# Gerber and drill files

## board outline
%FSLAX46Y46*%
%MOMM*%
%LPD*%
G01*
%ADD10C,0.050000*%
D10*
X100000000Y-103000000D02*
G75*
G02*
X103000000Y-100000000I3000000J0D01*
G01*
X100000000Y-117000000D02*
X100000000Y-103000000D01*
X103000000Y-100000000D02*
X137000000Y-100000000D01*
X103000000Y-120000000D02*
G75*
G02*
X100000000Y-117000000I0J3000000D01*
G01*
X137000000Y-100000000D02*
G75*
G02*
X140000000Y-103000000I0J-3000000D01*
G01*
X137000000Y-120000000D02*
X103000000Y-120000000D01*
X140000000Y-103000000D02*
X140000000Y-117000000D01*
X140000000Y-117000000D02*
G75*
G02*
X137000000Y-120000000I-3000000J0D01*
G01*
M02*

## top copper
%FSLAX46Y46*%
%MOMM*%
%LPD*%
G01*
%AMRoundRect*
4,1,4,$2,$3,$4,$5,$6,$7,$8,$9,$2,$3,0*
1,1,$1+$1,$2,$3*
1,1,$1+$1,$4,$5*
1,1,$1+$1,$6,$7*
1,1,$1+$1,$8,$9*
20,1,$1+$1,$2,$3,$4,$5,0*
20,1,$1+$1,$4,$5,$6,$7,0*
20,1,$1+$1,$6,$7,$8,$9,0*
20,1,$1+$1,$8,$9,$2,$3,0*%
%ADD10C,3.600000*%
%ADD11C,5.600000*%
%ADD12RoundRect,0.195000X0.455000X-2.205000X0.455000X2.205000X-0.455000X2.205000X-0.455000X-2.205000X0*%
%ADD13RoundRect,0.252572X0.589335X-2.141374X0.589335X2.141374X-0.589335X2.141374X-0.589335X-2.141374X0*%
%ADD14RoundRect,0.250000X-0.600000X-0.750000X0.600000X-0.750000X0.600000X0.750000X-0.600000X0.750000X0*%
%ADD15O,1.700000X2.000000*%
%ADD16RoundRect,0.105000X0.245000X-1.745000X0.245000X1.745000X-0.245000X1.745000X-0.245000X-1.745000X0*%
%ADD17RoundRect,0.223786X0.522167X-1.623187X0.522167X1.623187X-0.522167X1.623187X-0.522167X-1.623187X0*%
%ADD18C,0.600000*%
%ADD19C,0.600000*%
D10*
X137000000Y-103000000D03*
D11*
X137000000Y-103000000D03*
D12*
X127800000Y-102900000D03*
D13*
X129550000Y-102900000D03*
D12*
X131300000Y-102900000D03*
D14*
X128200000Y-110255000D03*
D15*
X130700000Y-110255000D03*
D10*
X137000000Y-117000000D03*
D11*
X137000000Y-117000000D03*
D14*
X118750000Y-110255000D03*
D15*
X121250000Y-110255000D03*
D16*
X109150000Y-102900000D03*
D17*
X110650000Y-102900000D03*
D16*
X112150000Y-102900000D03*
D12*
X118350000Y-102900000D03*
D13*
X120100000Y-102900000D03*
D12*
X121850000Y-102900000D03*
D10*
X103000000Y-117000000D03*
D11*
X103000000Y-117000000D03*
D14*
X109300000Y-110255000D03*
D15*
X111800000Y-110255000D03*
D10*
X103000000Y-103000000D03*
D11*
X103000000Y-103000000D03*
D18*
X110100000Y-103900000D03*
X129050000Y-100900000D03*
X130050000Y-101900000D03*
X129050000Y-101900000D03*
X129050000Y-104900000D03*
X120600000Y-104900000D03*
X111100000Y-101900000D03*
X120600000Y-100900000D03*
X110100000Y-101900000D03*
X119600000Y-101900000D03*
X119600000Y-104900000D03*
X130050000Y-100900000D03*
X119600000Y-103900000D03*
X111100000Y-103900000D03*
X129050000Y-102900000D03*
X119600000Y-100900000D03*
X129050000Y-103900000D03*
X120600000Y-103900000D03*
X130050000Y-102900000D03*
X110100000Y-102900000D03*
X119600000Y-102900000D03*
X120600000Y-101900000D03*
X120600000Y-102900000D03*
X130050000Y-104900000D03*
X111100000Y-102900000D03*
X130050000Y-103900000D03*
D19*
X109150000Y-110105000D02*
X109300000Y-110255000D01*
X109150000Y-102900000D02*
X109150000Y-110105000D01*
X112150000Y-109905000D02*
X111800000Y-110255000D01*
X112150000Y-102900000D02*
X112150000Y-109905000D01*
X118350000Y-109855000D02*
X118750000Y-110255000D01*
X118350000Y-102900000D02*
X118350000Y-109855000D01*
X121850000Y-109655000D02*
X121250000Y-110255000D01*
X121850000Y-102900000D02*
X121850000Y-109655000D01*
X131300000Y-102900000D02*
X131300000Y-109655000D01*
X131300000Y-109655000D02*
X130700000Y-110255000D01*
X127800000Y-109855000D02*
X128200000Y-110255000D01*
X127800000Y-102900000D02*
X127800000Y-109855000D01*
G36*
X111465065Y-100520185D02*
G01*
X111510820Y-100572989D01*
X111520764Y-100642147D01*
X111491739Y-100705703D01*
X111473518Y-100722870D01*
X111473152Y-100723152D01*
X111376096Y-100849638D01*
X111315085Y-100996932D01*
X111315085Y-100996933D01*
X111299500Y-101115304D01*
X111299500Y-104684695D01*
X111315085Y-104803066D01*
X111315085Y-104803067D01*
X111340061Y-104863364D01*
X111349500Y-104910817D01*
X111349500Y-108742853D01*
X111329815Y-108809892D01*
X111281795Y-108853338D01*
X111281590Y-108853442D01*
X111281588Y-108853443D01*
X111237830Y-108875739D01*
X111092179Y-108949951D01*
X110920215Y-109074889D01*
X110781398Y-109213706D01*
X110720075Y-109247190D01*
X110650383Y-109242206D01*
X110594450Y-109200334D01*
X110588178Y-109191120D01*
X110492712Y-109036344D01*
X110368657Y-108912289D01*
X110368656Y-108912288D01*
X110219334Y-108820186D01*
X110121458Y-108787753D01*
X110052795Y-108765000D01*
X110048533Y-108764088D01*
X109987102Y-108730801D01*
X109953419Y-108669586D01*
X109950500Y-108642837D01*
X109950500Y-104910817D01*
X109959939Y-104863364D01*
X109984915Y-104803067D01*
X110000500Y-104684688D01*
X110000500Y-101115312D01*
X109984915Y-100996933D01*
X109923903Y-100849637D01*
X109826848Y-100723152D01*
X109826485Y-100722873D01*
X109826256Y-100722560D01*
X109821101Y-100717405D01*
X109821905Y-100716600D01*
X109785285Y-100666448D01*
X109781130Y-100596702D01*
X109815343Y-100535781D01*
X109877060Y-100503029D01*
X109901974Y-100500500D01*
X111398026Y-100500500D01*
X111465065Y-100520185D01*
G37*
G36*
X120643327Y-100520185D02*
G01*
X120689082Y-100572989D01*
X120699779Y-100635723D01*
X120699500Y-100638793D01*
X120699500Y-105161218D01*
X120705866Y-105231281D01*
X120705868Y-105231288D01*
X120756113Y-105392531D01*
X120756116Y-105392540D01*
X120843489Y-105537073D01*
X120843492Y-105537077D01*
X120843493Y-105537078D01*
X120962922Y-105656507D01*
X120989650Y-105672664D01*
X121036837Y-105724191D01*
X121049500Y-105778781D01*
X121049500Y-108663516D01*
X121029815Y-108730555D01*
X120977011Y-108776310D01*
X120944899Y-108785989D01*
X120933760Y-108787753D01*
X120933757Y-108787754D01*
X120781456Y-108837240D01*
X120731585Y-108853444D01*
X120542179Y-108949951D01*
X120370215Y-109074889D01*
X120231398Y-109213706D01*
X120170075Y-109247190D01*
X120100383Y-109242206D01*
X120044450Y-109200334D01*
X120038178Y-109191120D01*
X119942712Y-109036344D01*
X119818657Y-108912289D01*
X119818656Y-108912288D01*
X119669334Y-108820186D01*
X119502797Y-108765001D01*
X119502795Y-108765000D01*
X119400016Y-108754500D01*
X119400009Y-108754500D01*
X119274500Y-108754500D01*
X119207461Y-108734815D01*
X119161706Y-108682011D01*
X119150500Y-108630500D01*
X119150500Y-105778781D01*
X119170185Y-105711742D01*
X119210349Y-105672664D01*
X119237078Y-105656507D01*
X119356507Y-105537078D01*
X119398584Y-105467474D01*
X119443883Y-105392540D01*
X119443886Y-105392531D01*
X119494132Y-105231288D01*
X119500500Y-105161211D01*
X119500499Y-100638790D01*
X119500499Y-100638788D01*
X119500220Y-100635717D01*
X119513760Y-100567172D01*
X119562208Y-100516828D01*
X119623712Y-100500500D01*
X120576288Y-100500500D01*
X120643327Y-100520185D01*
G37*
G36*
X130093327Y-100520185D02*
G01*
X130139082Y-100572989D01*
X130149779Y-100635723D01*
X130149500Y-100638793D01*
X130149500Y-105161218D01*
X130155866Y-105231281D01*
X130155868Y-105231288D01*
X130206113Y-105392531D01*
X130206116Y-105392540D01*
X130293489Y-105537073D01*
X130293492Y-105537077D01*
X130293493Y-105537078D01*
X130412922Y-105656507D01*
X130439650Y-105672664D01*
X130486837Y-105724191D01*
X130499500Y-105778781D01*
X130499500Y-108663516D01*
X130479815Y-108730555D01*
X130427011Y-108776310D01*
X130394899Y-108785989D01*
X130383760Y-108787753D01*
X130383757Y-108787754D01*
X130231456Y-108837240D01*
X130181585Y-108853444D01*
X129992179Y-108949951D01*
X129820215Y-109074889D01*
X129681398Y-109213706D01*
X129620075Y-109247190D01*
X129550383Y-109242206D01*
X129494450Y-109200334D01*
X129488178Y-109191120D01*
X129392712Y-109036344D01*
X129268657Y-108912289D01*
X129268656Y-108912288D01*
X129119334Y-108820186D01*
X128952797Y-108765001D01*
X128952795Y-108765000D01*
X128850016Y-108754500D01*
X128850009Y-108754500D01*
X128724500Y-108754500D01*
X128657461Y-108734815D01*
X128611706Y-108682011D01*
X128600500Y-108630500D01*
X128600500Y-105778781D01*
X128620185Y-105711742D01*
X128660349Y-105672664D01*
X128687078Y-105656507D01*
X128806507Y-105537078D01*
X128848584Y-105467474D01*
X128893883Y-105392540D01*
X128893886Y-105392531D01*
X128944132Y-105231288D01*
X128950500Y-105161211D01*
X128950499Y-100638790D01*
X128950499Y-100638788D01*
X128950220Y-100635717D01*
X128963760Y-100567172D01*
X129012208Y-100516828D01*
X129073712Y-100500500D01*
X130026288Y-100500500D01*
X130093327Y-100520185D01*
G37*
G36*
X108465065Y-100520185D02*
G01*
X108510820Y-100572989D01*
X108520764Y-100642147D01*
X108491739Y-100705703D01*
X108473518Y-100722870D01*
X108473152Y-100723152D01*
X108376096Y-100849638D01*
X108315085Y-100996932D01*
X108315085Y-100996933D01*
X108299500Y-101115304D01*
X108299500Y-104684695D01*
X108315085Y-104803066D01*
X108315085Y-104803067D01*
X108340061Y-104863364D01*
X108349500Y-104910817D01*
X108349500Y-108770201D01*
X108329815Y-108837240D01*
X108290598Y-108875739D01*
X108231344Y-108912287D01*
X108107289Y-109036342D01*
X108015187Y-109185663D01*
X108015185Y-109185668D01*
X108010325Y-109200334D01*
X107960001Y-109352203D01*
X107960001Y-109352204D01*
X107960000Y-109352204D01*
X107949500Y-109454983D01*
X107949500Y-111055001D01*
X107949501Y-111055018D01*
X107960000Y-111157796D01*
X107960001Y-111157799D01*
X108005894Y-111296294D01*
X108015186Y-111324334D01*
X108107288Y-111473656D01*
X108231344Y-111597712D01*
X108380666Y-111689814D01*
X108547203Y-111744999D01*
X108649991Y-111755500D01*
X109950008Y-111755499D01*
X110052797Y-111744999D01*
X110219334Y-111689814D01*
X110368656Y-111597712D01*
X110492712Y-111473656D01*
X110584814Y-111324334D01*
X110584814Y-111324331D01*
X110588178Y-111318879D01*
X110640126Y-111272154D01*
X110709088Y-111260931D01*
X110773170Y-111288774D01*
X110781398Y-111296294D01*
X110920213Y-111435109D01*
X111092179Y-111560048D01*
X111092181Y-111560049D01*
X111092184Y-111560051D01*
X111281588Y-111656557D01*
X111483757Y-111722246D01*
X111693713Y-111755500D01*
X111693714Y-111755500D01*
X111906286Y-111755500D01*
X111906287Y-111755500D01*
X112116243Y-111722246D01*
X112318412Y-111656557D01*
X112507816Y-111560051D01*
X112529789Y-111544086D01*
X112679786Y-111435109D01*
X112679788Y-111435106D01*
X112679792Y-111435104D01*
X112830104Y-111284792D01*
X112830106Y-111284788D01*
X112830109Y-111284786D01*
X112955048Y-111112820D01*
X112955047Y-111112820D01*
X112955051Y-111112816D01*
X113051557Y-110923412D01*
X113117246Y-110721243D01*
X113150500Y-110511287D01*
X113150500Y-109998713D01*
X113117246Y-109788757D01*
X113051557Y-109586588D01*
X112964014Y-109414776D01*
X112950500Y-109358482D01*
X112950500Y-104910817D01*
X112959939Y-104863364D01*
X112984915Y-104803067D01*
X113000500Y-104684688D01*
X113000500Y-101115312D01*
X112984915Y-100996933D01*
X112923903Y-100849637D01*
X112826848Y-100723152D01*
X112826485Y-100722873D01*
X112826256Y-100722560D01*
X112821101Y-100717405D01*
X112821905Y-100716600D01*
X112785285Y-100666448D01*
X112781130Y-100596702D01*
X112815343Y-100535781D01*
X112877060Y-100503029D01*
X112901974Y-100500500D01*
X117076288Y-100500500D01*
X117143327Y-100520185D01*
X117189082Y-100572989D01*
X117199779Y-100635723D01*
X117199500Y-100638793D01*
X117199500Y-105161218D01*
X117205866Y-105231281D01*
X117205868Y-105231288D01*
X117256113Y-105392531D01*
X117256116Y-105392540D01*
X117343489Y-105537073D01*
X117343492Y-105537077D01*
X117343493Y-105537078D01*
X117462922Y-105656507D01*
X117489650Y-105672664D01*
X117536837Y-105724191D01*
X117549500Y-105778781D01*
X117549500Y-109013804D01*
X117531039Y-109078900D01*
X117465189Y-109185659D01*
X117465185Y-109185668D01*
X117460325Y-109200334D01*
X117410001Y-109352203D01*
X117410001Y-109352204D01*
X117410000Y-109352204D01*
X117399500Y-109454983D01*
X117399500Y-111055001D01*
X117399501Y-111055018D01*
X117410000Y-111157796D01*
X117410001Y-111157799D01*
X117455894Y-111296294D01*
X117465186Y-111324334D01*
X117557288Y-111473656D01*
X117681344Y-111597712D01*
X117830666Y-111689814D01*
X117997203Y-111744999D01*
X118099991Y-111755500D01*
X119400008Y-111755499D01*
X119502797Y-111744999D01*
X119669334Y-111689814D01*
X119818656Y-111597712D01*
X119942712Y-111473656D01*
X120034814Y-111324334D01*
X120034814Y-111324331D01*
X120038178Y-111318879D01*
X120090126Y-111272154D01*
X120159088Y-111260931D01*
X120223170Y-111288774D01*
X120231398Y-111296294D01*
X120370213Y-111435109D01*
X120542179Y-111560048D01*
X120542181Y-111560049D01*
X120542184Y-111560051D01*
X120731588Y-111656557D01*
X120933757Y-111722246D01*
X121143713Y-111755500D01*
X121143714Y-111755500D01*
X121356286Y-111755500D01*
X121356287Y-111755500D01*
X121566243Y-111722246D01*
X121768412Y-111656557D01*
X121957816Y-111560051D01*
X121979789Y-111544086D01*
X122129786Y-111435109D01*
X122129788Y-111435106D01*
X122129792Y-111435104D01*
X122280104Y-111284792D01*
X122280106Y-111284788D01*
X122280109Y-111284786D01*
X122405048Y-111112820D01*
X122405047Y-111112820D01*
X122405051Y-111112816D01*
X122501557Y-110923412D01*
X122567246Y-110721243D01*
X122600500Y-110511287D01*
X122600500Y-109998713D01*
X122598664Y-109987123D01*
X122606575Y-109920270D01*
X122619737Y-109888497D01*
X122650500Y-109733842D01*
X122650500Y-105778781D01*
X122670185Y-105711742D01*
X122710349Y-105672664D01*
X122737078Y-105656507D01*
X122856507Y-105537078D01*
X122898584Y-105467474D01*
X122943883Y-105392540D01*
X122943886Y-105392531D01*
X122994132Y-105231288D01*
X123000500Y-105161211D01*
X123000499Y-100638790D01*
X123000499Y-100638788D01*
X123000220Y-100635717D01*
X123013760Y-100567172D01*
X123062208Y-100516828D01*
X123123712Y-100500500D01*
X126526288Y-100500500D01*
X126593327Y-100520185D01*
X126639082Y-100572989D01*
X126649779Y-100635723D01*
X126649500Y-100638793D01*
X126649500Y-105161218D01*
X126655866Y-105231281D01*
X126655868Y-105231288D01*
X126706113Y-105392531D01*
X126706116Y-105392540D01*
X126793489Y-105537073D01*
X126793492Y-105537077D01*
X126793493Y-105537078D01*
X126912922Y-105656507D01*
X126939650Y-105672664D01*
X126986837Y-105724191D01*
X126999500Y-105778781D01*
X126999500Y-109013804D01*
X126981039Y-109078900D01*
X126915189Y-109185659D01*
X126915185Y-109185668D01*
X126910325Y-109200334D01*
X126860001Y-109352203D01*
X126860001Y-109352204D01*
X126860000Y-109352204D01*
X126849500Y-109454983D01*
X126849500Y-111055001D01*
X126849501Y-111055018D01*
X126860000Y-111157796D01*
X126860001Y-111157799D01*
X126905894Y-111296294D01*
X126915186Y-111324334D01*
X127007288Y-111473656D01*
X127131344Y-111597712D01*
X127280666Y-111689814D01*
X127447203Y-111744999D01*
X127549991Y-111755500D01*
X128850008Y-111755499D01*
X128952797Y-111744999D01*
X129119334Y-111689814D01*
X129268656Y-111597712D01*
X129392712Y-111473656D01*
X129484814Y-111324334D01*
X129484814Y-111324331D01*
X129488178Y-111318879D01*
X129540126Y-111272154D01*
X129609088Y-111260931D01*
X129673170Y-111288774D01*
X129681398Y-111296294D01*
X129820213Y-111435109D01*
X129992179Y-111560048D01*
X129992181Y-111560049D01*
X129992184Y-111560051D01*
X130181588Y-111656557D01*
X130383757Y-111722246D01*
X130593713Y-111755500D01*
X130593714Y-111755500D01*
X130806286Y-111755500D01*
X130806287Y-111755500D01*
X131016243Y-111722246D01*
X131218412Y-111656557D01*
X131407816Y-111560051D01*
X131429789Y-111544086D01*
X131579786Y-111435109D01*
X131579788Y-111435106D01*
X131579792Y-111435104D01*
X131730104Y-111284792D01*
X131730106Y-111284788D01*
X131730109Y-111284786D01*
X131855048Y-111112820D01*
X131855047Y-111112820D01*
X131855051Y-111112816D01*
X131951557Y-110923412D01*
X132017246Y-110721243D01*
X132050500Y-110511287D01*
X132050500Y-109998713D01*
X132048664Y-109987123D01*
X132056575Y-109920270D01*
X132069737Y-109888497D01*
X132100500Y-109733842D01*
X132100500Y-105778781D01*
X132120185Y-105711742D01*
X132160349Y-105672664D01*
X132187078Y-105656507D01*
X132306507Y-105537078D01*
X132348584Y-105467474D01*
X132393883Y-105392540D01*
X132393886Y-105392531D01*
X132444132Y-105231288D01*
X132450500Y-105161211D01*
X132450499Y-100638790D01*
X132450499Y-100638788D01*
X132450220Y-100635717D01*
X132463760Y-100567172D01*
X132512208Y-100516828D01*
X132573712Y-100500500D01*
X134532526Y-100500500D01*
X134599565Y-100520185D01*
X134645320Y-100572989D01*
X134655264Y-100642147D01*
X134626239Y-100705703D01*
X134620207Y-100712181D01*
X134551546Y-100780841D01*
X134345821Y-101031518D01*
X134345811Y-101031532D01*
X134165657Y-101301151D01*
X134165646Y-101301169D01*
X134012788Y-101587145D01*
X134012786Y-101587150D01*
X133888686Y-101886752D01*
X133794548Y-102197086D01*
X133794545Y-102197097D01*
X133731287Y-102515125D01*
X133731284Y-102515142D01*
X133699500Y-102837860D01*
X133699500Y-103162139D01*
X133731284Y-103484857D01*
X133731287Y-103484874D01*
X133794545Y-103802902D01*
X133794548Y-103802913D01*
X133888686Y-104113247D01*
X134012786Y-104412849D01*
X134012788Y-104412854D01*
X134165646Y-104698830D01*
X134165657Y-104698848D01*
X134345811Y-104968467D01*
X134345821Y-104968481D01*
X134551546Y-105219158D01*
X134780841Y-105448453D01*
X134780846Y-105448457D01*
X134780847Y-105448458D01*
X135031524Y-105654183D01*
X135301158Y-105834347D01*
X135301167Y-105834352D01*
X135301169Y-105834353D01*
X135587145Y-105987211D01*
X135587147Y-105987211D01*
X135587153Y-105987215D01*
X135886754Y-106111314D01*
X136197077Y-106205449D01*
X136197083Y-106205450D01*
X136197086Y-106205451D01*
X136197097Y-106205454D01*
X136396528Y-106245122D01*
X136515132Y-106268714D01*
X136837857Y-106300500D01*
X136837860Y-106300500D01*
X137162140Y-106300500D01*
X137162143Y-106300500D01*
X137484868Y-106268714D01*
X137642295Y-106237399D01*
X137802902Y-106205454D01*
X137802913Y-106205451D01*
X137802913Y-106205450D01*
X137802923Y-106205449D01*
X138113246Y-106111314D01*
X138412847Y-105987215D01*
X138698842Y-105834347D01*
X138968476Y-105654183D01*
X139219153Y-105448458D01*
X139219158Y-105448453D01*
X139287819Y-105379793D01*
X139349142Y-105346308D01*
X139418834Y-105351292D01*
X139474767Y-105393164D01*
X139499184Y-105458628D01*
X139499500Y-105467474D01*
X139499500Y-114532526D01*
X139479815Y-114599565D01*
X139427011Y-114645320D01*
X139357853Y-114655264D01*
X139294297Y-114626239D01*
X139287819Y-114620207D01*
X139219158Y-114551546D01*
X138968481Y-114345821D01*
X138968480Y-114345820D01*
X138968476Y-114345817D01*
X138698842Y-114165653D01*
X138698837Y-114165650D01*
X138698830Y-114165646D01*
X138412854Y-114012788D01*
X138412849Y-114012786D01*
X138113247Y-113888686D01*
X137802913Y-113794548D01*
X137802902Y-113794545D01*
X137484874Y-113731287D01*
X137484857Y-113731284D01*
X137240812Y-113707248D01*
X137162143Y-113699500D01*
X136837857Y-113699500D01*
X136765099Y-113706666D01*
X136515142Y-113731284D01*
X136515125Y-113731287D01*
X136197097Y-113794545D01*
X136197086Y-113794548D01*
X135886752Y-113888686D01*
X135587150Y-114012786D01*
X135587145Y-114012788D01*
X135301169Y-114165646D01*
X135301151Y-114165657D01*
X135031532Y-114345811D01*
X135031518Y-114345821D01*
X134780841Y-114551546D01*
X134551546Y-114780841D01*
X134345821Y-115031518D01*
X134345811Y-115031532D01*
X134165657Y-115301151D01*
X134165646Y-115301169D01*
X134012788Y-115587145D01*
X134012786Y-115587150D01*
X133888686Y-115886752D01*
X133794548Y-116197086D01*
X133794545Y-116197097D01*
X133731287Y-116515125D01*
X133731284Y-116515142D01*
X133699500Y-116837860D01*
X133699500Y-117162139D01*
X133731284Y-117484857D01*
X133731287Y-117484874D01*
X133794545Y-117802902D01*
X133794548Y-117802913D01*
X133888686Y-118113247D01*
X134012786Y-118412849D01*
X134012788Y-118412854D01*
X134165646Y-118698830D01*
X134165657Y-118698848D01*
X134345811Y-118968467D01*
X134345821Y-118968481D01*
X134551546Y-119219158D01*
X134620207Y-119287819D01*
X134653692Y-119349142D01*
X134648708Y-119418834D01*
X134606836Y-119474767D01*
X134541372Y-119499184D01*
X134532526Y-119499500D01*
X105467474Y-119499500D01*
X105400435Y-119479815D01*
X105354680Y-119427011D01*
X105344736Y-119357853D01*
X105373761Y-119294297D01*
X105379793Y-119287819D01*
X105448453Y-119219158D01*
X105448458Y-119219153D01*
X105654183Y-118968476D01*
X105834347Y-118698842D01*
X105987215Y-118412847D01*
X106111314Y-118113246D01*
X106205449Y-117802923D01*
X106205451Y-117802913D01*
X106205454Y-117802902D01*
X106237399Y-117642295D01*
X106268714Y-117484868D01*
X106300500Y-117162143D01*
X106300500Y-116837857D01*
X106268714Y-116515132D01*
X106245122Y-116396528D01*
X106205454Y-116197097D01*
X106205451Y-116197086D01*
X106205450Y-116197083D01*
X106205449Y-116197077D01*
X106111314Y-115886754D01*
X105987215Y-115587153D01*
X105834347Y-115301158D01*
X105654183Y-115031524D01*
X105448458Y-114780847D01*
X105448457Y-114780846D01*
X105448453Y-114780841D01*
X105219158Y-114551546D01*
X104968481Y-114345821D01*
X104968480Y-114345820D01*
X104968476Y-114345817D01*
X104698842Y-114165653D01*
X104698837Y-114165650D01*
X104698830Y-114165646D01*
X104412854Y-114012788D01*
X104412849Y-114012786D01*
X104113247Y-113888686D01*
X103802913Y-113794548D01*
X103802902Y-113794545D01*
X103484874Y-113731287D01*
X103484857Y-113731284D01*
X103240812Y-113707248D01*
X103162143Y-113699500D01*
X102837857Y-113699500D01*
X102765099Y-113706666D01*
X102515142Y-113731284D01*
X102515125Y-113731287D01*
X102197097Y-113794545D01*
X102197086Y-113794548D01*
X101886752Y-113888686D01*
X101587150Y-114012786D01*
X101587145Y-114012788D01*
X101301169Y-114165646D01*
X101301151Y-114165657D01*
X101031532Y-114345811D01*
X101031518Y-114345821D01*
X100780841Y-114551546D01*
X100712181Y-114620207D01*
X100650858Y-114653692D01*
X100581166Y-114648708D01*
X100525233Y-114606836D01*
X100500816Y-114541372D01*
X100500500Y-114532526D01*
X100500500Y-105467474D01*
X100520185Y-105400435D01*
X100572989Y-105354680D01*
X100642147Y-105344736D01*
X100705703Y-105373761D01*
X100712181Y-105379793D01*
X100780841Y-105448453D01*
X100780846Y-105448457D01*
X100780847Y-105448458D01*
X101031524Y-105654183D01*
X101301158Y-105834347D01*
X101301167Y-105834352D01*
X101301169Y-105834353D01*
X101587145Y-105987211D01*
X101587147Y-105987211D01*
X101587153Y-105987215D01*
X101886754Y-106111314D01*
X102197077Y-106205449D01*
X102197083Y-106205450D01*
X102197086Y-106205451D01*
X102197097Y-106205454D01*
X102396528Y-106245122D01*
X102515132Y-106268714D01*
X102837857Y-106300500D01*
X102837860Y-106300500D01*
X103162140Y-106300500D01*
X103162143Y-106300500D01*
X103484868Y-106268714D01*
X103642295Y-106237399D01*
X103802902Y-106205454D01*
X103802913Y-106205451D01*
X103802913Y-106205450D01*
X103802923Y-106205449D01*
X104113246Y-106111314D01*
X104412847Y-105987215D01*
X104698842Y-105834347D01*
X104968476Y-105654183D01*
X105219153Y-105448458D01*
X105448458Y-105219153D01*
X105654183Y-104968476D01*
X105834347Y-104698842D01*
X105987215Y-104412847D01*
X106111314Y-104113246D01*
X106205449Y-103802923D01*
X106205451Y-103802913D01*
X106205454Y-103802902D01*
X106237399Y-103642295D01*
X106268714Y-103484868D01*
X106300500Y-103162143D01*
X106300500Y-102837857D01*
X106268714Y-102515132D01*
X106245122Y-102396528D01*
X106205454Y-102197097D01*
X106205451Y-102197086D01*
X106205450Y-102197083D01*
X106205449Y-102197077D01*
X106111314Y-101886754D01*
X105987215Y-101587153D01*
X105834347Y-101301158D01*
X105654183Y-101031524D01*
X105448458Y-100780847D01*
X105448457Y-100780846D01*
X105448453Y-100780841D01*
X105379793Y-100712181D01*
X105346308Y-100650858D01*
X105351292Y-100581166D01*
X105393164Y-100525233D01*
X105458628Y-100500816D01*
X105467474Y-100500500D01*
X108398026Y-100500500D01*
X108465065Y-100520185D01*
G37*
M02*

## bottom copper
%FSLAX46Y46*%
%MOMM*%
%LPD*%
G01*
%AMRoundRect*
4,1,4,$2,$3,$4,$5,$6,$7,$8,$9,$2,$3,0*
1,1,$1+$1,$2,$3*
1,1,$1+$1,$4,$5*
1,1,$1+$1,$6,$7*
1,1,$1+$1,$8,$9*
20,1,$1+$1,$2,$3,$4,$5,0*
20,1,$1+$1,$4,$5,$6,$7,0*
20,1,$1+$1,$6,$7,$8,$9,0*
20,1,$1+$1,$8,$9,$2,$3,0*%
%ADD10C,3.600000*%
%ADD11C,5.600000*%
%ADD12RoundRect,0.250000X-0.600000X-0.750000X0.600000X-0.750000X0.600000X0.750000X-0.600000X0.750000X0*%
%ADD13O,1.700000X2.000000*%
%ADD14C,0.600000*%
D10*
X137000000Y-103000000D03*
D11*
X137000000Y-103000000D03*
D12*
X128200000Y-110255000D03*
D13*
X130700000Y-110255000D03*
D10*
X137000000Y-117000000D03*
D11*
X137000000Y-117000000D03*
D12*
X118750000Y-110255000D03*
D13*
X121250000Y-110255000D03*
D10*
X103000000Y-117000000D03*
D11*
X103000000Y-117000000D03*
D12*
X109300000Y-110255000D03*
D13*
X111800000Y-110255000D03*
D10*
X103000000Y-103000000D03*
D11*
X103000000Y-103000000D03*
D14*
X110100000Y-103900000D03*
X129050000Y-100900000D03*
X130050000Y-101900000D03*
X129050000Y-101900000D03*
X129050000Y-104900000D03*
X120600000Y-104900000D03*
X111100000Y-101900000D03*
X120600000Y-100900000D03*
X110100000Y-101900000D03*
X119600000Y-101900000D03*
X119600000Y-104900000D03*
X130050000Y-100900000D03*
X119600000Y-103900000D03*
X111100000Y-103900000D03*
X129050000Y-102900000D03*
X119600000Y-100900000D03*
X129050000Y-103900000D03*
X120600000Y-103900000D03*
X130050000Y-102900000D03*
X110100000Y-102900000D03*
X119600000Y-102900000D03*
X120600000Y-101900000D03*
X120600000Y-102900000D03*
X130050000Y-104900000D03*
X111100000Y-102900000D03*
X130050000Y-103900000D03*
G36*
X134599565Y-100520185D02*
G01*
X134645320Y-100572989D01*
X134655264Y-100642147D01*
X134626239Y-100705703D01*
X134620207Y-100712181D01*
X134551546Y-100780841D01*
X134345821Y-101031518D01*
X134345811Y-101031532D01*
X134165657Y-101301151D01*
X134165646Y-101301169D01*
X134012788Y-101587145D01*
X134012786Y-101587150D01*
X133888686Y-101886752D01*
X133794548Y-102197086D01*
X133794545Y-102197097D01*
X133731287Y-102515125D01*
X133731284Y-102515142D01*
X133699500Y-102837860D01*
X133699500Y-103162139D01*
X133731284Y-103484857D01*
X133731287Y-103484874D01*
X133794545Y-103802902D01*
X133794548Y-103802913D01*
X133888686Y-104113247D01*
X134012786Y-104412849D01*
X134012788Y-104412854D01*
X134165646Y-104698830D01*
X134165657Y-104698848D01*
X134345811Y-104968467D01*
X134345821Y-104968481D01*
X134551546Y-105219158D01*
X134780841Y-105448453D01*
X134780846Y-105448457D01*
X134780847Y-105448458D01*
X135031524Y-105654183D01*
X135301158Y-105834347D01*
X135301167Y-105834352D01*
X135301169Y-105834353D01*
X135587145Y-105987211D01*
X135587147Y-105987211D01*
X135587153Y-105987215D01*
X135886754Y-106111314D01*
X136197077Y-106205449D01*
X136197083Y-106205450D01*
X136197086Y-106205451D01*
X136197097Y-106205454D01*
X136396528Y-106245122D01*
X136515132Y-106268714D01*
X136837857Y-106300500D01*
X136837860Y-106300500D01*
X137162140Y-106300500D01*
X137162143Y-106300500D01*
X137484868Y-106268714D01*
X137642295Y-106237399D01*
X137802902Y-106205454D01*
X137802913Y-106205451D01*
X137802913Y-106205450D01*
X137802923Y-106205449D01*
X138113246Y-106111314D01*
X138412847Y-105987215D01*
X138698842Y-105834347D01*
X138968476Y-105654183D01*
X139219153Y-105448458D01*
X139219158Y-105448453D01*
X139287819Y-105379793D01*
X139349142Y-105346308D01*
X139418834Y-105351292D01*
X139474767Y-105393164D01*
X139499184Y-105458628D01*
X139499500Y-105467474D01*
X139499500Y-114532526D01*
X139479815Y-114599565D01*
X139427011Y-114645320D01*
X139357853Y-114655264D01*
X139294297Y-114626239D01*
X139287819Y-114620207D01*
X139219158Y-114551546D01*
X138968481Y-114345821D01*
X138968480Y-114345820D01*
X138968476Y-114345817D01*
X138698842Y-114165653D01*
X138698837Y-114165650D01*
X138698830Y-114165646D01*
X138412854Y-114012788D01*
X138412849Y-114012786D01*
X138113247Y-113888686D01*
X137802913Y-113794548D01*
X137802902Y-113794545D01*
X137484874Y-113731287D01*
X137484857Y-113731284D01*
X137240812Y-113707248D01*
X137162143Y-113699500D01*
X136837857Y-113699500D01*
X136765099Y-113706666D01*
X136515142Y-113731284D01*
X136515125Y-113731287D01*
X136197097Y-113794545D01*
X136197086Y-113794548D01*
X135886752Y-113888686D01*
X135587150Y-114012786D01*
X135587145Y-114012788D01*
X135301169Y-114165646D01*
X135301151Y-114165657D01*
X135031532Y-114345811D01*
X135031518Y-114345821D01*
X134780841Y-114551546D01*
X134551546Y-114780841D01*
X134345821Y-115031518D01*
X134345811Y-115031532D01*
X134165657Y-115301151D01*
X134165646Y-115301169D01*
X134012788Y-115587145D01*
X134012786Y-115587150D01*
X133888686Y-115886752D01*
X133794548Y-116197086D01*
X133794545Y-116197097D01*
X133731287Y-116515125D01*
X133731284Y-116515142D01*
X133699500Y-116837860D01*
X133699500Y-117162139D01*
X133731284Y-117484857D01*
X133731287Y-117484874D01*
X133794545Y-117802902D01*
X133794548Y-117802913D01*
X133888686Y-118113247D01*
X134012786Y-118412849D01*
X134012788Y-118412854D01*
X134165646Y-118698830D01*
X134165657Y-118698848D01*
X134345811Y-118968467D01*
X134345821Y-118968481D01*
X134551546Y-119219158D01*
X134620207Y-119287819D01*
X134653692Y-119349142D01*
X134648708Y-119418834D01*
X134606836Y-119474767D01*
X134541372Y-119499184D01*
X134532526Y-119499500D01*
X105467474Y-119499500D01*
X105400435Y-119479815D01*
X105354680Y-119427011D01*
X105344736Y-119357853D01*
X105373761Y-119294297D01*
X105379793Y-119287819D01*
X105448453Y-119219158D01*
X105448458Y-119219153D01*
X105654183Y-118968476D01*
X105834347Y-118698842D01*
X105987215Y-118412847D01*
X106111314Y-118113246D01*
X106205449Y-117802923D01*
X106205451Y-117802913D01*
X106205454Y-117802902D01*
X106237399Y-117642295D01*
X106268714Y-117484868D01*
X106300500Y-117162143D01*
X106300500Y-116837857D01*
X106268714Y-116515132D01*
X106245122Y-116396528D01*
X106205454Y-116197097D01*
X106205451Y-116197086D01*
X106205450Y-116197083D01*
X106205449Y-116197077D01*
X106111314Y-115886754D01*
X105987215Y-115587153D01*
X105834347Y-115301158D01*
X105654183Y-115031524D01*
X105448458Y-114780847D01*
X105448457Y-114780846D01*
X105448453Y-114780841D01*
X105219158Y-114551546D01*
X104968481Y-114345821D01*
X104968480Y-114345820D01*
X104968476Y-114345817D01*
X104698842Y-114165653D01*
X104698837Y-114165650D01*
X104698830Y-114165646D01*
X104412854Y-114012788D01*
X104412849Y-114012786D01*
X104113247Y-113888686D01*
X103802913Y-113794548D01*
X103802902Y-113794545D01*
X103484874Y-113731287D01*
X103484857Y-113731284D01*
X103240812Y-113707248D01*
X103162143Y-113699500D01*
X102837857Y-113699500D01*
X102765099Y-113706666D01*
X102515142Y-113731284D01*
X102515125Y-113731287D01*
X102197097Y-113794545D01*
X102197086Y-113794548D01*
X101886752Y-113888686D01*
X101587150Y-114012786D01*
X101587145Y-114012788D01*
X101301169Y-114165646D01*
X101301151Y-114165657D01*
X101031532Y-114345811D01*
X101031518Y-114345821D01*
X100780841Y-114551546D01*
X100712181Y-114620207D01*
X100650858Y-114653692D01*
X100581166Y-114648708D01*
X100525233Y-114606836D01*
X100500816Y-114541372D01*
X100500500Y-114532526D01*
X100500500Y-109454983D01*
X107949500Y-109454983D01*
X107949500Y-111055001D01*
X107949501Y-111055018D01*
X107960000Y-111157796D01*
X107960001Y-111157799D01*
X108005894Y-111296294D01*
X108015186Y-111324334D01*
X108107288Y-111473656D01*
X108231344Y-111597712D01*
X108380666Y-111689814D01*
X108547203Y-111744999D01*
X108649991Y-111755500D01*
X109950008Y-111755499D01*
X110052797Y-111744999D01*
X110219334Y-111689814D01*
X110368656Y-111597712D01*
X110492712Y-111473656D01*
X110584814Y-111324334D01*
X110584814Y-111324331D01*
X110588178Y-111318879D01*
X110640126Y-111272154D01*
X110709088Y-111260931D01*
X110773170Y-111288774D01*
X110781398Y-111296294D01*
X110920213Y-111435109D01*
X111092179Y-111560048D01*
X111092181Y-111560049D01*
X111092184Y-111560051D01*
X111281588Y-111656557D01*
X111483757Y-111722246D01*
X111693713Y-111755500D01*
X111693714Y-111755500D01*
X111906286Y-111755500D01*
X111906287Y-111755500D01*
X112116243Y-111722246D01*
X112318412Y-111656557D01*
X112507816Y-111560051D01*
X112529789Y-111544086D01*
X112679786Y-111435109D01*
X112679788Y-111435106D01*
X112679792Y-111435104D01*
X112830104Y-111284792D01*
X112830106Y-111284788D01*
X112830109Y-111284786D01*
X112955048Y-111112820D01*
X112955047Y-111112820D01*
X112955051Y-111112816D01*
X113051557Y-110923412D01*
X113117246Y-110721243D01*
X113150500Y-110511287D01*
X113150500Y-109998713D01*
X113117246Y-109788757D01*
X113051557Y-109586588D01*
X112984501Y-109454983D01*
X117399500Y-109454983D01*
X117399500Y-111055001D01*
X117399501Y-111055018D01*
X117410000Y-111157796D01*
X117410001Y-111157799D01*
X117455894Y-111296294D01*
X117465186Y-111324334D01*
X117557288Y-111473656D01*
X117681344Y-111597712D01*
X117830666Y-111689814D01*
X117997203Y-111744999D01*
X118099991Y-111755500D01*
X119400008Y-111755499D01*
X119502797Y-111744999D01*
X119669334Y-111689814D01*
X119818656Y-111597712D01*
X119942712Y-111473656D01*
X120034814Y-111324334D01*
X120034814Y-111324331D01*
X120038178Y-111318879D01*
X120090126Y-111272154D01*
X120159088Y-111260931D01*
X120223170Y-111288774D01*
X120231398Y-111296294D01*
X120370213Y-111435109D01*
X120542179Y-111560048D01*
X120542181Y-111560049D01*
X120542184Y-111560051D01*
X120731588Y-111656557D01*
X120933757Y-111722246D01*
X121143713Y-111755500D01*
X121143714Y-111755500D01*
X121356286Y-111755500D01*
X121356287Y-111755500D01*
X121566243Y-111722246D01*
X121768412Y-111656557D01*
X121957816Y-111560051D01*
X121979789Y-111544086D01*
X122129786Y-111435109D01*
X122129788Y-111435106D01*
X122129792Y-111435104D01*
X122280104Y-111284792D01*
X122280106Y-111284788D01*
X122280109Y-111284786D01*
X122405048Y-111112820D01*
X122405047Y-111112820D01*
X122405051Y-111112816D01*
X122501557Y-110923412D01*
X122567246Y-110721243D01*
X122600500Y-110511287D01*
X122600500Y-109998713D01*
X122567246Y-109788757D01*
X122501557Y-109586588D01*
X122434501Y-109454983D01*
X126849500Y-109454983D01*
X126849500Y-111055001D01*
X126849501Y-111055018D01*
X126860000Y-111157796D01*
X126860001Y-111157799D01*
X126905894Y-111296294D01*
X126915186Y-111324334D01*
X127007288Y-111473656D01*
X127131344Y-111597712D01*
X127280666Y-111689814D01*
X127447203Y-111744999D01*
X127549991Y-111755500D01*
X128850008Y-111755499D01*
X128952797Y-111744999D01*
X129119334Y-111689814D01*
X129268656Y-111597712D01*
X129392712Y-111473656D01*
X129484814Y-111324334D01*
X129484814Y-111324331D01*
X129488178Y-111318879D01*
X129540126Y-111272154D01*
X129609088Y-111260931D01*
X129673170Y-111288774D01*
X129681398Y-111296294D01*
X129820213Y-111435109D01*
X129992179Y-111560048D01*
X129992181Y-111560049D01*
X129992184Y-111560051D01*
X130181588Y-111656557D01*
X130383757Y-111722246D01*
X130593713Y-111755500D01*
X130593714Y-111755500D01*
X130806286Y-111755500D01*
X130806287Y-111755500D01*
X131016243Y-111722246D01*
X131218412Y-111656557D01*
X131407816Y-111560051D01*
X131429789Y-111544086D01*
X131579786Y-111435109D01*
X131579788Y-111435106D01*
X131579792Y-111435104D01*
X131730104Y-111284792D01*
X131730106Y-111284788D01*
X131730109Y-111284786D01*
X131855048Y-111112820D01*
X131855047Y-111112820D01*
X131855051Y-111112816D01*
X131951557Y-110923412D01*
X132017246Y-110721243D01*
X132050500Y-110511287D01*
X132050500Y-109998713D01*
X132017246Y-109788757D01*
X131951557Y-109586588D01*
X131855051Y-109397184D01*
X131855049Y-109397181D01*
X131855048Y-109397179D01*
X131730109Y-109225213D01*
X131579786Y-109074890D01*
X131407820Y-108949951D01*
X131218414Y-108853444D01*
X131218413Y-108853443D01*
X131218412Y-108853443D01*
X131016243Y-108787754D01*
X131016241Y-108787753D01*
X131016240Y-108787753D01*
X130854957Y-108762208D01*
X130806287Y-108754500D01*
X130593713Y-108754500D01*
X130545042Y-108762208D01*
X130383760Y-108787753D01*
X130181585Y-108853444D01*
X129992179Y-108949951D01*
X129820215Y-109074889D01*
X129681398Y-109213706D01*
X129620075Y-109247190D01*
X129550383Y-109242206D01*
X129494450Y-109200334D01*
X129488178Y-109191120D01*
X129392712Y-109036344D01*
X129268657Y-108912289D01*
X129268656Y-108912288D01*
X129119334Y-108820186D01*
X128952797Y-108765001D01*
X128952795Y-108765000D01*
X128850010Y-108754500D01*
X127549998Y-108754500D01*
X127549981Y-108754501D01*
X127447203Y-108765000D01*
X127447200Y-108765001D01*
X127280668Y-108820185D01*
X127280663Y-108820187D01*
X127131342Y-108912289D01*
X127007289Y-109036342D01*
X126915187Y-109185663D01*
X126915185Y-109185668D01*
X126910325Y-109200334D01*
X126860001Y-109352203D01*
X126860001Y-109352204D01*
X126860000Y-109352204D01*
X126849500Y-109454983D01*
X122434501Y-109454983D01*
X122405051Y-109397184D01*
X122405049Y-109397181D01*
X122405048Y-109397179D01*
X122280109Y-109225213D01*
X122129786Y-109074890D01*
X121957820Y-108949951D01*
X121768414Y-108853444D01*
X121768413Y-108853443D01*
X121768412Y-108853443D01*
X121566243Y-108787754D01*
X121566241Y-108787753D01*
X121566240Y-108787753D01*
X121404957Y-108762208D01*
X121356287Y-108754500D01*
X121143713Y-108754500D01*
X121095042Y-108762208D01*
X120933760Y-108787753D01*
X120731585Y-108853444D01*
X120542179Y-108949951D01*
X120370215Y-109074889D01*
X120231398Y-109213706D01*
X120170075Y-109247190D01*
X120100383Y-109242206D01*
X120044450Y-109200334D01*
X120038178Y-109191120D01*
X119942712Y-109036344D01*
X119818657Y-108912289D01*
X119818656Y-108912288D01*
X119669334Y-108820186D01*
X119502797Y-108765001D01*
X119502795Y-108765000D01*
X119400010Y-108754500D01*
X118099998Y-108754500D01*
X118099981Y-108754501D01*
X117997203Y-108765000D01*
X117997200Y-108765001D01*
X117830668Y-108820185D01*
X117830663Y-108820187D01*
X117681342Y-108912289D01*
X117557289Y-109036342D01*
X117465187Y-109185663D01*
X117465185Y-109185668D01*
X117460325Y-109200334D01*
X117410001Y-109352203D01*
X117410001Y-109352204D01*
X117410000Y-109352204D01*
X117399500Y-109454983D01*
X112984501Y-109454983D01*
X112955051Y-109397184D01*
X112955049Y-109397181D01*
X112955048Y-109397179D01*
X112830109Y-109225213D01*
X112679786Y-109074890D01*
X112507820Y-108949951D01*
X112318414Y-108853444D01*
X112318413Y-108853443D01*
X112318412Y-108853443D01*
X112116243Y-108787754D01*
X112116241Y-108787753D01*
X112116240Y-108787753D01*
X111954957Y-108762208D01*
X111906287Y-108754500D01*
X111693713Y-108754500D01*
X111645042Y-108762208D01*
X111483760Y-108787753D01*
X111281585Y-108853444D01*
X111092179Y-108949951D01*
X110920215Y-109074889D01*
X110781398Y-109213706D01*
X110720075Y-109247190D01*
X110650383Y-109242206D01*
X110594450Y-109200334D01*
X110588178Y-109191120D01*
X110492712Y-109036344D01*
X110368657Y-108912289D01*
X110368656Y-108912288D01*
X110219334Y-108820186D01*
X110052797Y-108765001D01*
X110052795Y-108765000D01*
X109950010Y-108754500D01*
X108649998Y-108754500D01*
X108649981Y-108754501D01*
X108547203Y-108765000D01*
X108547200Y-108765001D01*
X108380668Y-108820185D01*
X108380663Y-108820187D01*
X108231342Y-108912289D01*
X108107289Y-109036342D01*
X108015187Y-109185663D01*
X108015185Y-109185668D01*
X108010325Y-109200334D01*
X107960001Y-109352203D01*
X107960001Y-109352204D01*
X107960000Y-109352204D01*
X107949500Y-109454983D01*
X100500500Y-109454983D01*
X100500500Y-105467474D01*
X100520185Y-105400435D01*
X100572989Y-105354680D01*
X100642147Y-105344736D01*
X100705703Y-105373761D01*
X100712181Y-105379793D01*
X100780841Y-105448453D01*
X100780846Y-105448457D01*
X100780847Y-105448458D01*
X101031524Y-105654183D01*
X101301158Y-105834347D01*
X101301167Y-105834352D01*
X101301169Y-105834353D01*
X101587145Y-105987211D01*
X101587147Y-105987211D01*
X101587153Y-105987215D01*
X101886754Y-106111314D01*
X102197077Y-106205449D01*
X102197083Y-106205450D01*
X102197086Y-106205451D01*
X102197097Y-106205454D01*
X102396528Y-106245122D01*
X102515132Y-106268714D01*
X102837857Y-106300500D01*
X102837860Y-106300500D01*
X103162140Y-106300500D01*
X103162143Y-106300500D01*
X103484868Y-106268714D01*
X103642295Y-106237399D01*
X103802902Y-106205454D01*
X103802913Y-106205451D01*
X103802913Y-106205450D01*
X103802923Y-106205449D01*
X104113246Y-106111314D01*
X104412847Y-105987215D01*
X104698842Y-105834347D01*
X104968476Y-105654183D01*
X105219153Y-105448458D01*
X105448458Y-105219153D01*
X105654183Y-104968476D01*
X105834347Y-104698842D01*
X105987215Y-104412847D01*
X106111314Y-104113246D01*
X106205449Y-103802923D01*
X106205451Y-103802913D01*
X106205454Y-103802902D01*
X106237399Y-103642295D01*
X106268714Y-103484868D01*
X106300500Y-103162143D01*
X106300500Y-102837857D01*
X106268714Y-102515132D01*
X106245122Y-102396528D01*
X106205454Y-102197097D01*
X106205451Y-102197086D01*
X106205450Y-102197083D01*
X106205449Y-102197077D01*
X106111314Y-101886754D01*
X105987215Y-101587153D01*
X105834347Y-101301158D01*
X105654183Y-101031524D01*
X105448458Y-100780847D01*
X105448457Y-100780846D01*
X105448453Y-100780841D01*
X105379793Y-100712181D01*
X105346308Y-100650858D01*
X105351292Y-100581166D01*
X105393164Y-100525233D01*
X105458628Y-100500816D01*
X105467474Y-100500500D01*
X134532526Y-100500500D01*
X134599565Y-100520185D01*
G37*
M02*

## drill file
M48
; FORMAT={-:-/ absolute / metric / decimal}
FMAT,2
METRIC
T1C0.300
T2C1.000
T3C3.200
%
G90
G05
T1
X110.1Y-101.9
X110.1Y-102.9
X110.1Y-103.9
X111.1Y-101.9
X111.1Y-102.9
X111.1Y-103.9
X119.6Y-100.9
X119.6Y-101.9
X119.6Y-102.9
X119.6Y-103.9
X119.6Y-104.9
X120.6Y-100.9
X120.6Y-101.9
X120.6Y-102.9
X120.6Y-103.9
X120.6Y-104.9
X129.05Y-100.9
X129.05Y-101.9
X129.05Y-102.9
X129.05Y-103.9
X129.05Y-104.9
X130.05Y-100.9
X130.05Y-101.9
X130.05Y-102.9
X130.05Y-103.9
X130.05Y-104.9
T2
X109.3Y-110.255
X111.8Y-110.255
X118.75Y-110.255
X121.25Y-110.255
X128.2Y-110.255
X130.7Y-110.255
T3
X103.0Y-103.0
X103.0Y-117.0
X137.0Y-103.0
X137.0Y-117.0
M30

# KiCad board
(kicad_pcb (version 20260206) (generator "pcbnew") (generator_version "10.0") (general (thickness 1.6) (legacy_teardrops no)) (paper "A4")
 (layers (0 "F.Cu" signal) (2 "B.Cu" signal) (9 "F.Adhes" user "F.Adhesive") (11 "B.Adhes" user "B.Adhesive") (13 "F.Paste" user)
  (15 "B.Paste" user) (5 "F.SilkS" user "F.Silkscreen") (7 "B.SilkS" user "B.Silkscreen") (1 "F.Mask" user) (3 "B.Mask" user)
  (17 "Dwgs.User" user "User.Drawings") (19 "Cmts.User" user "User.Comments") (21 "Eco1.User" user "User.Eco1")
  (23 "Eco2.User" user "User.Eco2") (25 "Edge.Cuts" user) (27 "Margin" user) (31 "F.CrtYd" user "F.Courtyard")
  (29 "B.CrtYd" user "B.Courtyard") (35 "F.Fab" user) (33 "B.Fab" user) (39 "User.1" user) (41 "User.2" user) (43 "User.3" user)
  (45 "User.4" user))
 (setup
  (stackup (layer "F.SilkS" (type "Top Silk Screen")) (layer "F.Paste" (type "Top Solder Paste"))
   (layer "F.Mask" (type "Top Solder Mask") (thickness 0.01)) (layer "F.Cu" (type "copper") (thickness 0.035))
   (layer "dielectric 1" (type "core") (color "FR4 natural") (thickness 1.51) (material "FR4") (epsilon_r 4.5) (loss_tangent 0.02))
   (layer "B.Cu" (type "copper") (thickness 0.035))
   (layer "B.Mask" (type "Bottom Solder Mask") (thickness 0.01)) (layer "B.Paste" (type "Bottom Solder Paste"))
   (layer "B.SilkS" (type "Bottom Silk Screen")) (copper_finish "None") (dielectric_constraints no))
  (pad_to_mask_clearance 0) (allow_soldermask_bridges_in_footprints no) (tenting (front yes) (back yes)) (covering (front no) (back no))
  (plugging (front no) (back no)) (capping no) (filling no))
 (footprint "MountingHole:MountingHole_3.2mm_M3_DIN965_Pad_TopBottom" (layer "F.Cu") (at 137 103)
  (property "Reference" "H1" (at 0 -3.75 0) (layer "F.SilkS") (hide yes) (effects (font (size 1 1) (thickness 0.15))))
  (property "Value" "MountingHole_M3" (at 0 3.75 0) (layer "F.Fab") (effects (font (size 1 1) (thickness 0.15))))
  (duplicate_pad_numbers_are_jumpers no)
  (pad "1" thru_hole circle (at 0 0) (size 3.6 3.6) (drill 3.2) (layers "*.Cu" "*.Mask") (remove_unused_layers no) (zone_connect 2))
  (pad "1" connect circle (at 0 0) (size 5.6 5.6) (layers "F.Cu" "F.Mask") (zone_connect 2))
  (pad "1" connect circle (at 0 0) (size 5.6 5.6) (layers "B.Cu" "B.Mask") (zone_connect 2)))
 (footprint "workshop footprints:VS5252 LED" (layer "F.Cu") (at 127.25 105.2 90)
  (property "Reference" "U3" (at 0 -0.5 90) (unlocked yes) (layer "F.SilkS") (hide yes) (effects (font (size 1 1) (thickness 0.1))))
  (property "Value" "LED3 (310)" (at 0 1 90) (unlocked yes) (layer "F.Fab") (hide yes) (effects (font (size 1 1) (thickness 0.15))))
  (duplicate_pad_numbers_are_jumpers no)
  (pad "1" smd roundrect (at 2.3 0.55 90) (size 4.8 1.3) (layers "F.Cu" "F.Mask" "F.Paste") (roundrect_rratio 0.15) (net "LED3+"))
  (pad "2" smd roundrect (at 2.3 2.3 90) (size 4.787892 1.683814) (layers "F.Cu" "F.Mask" "F.Paste") (roundrect_rratio 0.15) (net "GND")
   (zone_connect 2))
  (pad "3" smd roundrect (at 2.3 4.05 90) (size 4.8 1.3) (layers "F.Cu" "F.Mask" "F.Paste") (roundrect_rratio 0.15) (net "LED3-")))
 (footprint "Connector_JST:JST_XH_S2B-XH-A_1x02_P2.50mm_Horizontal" (layer "F.Cu") (at 128.2 110.255)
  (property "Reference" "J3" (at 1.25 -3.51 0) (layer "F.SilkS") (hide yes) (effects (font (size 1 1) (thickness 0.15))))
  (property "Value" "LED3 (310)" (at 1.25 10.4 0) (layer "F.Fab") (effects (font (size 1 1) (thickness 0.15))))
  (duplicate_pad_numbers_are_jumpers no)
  (pad "1" thru_hole roundrect (at 0 0) (size 1.7 2) (drill 1) (layers "*.Cu" "*.Mask") (remove_unused_layers no)
   (roundrect_rratio 0.147059) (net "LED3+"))
  (pad "2" thru_hole oval (at 2.5 0) (size 1.7 2) (drill 1) (layers "*.Cu" "*.Mask") (remove_unused_layers no) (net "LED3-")))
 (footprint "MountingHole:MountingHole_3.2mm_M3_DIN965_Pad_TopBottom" (layer "F.Cu") (at 137 117)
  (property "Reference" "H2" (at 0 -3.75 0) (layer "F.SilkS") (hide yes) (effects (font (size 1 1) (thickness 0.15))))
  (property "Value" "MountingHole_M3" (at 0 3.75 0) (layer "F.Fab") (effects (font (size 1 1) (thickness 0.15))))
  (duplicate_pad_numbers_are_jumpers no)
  (pad "1" thru_hole circle (at 0 0) (size 3.6 3.6) (drill 3.2) (layers "*.Cu" "*.Mask") (remove_unused_layers no) (zone_connect 2))
  (pad "1" connect circle (at 0 0) (size 5.6 5.6) (layers "F.Cu" "F.Mask") (zone_connect 2))
  (pad "1" connect circle (at 0 0) (size 5.6 5.6) (layers "B.Cu" "B.Mask") (zone_connect 2)))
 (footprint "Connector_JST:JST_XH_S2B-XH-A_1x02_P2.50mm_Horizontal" (layer "F.Cu") (at 118.75 110.255)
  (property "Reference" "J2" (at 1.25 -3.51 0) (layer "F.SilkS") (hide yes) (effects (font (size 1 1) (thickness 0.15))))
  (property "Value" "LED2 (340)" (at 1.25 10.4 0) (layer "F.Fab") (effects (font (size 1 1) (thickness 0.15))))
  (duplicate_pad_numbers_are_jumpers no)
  (pad "1" thru_hole roundrect (at 0 0) (size 1.7 2) (drill 1) (layers "*.Cu" "*.Mask") (remove_unused_layers no)
   (roundrect_rratio 0.147059) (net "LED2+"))
  (pad "2" thru_hole oval (at 2.5 0) (size 1.7 2) (drill 1) (layers "*.Cu" "*.Mask") (remove_unused_layers no) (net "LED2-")))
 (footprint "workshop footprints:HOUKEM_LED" (layer "F.Cu") (at 108.9 104.65 90)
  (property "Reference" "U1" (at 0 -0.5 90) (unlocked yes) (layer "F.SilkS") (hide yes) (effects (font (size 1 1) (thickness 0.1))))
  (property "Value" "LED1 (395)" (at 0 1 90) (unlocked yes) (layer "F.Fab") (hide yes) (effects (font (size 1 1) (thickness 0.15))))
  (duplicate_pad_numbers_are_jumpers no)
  (pad "1" smd roundrect (at 1.75 0.25 90) (size 3.7 0.7) (layers "F.Cu" "F.Mask" "F.Paste") (roundrect_rratio 0.15) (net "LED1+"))
  (pad "2" smd roundrect (at 1.75 1.75 90) (size 3.693946 1.491907) (layers "F.Cu" "F.Mask" "F.Paste") (roundrect_rratio 0.15) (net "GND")
   (zone_connect 2))
  (pad "3" smd roundrect (at 1.75 3.25 90) (size 3.7 0.7) (layers "F.Cu" "F.Mask" "F.Paste") (roundrect_rratio 0.15) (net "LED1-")))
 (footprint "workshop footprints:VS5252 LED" (layer "F.Cu") (at 117.8 105.2 90)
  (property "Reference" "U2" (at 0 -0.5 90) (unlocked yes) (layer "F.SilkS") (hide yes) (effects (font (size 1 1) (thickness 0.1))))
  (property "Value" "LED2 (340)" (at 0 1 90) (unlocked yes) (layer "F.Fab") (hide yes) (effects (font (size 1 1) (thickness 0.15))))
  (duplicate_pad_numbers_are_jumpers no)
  (pad "1" smd roundrect (at 2.3 0.55 90) (size 4.8 1.3) (layers "F.Cu" "F.Mask" "F.Paste") (roundrect_rratio 0.15) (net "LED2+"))
  (pad "2" smd roundrect (at 2.3 2.3 90) (size 4.787892 1.683814) (layers "F.Cu" "F.Mask" "F.Paste") (roundrect_rratio 0.15) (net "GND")
   (zone_connect 2))
  (pad "3" smd roundrect (at 2.3 4.05 90) (size 4.8 1.3) (layers "F.Cu" "F.Mask" "F.Paste") (roundrect_rratio 0.15) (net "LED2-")))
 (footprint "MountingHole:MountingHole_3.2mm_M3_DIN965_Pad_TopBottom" (layer "F.Cu") (at 103 117)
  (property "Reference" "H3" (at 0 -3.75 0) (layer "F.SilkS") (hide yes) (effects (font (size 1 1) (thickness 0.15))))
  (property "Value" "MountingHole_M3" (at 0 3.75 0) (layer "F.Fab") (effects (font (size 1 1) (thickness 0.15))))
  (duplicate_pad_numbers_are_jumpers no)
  (pad "1" thru_hole circle (at 0 0) (size 3.6 3.6) (drill 3.2) (layers "*.Cu" "*.Mask") (remove_unused_layers no) (zone_connect 2))
  (pad "1" connect circle (at 0 0) (size 5.6 5.6) (layers "F.Cu" "F.Mask") (zone_connect 2))
  (pad "1" connect circle (at 0 0) (size 5.6 5.6) (layers "B.Cu" "B.Mask") (zone_connect 2)))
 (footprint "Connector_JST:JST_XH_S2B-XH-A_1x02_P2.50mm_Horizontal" (layer "F.Cu") (at 109.3 110.255)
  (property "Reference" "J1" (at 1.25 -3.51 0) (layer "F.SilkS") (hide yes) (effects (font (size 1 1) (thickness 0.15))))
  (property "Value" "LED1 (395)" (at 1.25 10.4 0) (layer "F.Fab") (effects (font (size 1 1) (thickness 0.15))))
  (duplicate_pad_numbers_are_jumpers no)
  (pad "1" thru_hole roundrect (at 0 0) (size 1.7 2) (drill 1) (layers "*.Cu" "*.Mask") (remove_unused_layers no)
   (roundrect_rratio 0.147059) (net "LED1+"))
  (pad "2" thru_hole oval (at 2.5 0) (size 1.7 2) (drill 1) (layers "*.Cu" "*.Mask") (remove_unused_layers no) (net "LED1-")))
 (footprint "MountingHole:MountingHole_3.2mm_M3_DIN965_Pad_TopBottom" (layer "F.Cu") (at 103 103)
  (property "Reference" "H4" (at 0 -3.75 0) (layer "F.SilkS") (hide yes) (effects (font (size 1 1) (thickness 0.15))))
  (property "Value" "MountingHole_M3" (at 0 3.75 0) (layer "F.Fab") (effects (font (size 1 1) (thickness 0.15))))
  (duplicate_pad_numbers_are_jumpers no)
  (pad "1" thru_hole circle (at 0 0) (size 3.6 3.6) (drill 3.2) (layers "*.Cu" "*.Mask") (remove_unused_layers no) (zone_connect 2))
  (pad "1" connect circle (at 0 0) (size 5.6 5.6) (layers "F.Cu" "F.Mask") (zone_connect 2))
  (pad "1" connect circle (at 0 0) (size 5.6 5.6) (layers "B.Cu" "B.Mask") (zone_connect 2)))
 (gr_arc (start 100 103) (mid 100.87868 100.87868) (end 103 100) (stroke (width 0.05) (type default)) (layer "Edge.Cuts"))
 (gr_line (start 100 117) (end 100 103) (stroke (width 0.05) (type default)) (layer "Edge.Cuts"))
 (gr_line (start 103 100) (end 137 100) (stroke (width 0.05) (type default)) (layer "Edge.Cuts"))
 (gr_arc (start 103 120) (mid 100.87868 119.12132) (end 100 117) (stroke (width 0.05) (type default)) (layer "Edge.Cuts"))
 (gr_arc (start 137 100) (mid 139.12132 100.87868) (end 140 103) (stroke (width 0.05) (type default)) (layer "Edge.Cuts"))
 (gr_line (start 137 120) (end 103 120) (stroke (width 0.05) (type default)) (layer "Edge.Cuts"))
 (gr_line (start 140 103) (end 140 117) (stroke (width 0.05) (type default)) (layer "Edge.Cuts"))
 (gr_arc (start 140 117) (mid 139.12132 119.12132) (end 137 120) (stroke (width 0.05) (type default)) (layer "Edge.Cuts"))
 (segment (start 109.15 110.105) (end 109.3 110.255) (width 0.6) (layer "F.Cu") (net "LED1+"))
 (segment (start 109.15 102.9) (end 109.15 110.105) (width 0.6) (layer "F.Cu") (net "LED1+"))
 (segment (start 112.15 109.905) (end 111.8 110.255) (width 0.6) (layer "F.Cu") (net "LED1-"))
 (segment (start 112.15 102.9) (end 112.15 109.905) (width 0.6) (layer "F.Cu") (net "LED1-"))
 (segment (start 118.35 109.855) (end 118.75 110.255) (width 0.6) (layer "F.Cu") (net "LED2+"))
 (segment (start 118.35 102.9) (end 118.35 109.855) (width 0.6) (layer "F.Cu") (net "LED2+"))
 (segment (start 121.85 109.655) (end 121.25 110.255) (width 0.6) (layer "F.Cu") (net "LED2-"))
 (segment (start 121.85 102.9) (end 121.85 109.655) (width 0.6) (layer "F.Cu") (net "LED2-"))
 (segment (start 131.3 102.9) (end 131.3 109.655) (width 0.6) (layer "F.Cu") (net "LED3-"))
 (segment (start 131.3 109.655) (end 130.7 110.255) (width 0.6) (layer "F.Cu") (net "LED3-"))
 (segment (start 127.8 109.855) (end 128.2 110.255) (width 0.6) (layer "F.Cu") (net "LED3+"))
 (segment (start 127.8 102.9) (end 127.8 109.855) (width 0.6) (layer "F.Cu") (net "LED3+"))
 (via (at 110.1 103.9) (size 0.6) (drill 0.3) (layers "F.Cu" "B.Cu") (capping no) (covering (front no) (back no))
  (plugging (front no) (back no)) (filling no) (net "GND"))
 (via (at 129.05 100.9) (size 0.6) (drill 0.3) (layers "F.Cu" "B.Cu") (capping no) (covering (front no) (back no))
  (plugging (front no) (back no)) (filling no) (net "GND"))
 (via (at 130.05 101.9) (size 0.6) (drill 0.3) (layers "F.Cu" "B.Cu") (capping no) (covering (front no) (back no))
  (plugging (front no) (back no)) (filling no) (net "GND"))
 (via (at 129.05 101.9) (size 0.6) (drill 0.3) (layers "F.Cu" "B.Cu") (capping no) (covering (front no) (back no))
  (plugging (front no) (back no)) (filling no) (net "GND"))
 (via (at 129.05 104.9) (size 0.6) (drill 0.3) (layers "F.Cu" "B.Cu") (capping no) (covering (front no) (back no))
  (plugging (front no) (back no)) (filling no) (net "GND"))
 (via (at 120.6 104.9) (size 0.6) (drill 0.3) (layers "F.Cu" "B.Cu") (capping no) (covering (front no) (back no))
  (plugging (front no) (back no)) (filling no) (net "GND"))
 (via (at 111.1 101.9) (size 0.6) (drill 0.3) (layers "F.Cu" "B.Cu") (capping no) (covering (front no) (back no))
  (plugging (front no) (back no)) (filling no) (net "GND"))
 (via (at 120.6 100.9) (size 0.6) (drill 0.3) (layers "F.Cu" "B.Cu") (capping no) (covering (front no) (back no))
  (plugging (front no) (back no)) (filling no) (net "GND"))
 (via (at 110.1 101.9) (size 0.6) (drill 0.3) (layers "F.Cu" "B.Cu") (capping no) (covering (front no) (back no))
  (plugging (front no) (back no)) (filling no) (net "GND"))
 (via (at 119.6 101.9) (size 0.6) (drill 0.3) (layers "F.Cu" "B.Cu") (capping no) (covering (front no) (back no))
  (plugging (front no) (back no)) (filling no) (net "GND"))
 (via (at 119.6 104.9) (size 0.6) (drill 0.3) (layers "F.Cu" "B.Cu") (capping no) (covering (front no) (back no))
  (plugging (front no) (back no)) (filling no) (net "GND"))
 (via (at 130.05 100.9) (size 0.6) (drill 0.3) (layers "F.Cu" "B.Cu") (capping no) (covering (front no) (back no))
  (plugging (front no) (back no)) (filling no) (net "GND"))
 (via (at 119.6 103.9) (size 0.6) (drill 0.3) (layers "F.Cu" "B.Cu") (capping no) (covering (front no) (back no))
  (plugging (front no) (back no)) (filling no) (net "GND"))
 (via (at 111.1 103.9) (size 0.6) (drill 0.3) (layers "F.Cu" "B.Cu") (capping no) (covering (front no) (back no))
  (plugging (front no) (back no)) (filling no) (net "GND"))
 (via (at 129.05 102.9) (size 0.6) (drill 0.3) (layers "F.Cu" "B.Cu") (capping no) (covering (front no) (back no))
  (plugging (front no) (back no)) (filling no) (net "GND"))
 (via (at 119.6 100.9) (size 0.6) (drill 0.3) (layers "F.Cu" "B.Cu") (capping no) (covering (front no) (back no))
  (plugging (front no) (back no)) (filling no) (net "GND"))
 (via (at 129.05 103.9) (size 0.6) (drill 0.3) (layers "F.Cu" "B.Cu") (capping no) (covering (front no) (back no))
  (plugging (front no) (back no)) (filling no) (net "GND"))
 (via (at 120.6 103.9) (size 0.6) (drill 0.3) (layers "F.Cu" "B.Cu") (capping no) (covering (front no) (back no))
  (plugging (front no) (back no)) (filling no) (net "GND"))
 (via (at 130.05 102.9) (size 0.6) (drill 0.3) (layers "F.Cu" "B.Cu") (capping no) (covering (front no) (back no))
  (plugging (front no) (back no)) (filling no) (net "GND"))
 (via (at 110.1 102.9) (size 0.6) (drill 0.3) (layers "F.Cu" "B.Cu") (capping no) (covering (front no) (back no))
  (plugging (front no) (back no)) (filling no) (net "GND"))
 (via (at 119.6 102.9) (size 0.6) (drill 0.3) (layers "F.Cu" "B.Cu") (capping no) (covering (front no) (back no))
  (plugging (front no) (back no)) (filling no) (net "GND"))
 (via (at 120.6 101.9) (size 0.6) (drill 0.3) (layers "F.Cu" "B.Cu") (capping no) (covering (front no) (back no))
  (plugging (front no) (back no)) (filling no) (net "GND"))
 (via (at 120.6 102.9) (size 0.6) (drill 0.3) (layers "F.Cu" "B.Cu") (capping no) (covering (front no) (back no))
  (plugging (front no) (back no)) (filling no) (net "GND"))
 (via (at 130.05 104.9) (size 0.6) (drill 0.3) (layers "F.Cu" "B.Cu") (capping no) (covering (front no) (back no))
  (plugging (front no) (back no)) (filling no) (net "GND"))
 (via (at 111.1 102.9) (size 0.6) (drill 0.3) (layers "F.Cu" "B.Cu") (capping no) (covering (front no) (back no))
  (plugging (front no) (back no)) (filling no) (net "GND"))
 (via (at 130.05 103.9) (size 0.6) (drill 0.3) (layers "F.Cu" "B.Cu") (capping no) (covering (front no) (back no))
  (plugging (front no) (back no)) (filling no) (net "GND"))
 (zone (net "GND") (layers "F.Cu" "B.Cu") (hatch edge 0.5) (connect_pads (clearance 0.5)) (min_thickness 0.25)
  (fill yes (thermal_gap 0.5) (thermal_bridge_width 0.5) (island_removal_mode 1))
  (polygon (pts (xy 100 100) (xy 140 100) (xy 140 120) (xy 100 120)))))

